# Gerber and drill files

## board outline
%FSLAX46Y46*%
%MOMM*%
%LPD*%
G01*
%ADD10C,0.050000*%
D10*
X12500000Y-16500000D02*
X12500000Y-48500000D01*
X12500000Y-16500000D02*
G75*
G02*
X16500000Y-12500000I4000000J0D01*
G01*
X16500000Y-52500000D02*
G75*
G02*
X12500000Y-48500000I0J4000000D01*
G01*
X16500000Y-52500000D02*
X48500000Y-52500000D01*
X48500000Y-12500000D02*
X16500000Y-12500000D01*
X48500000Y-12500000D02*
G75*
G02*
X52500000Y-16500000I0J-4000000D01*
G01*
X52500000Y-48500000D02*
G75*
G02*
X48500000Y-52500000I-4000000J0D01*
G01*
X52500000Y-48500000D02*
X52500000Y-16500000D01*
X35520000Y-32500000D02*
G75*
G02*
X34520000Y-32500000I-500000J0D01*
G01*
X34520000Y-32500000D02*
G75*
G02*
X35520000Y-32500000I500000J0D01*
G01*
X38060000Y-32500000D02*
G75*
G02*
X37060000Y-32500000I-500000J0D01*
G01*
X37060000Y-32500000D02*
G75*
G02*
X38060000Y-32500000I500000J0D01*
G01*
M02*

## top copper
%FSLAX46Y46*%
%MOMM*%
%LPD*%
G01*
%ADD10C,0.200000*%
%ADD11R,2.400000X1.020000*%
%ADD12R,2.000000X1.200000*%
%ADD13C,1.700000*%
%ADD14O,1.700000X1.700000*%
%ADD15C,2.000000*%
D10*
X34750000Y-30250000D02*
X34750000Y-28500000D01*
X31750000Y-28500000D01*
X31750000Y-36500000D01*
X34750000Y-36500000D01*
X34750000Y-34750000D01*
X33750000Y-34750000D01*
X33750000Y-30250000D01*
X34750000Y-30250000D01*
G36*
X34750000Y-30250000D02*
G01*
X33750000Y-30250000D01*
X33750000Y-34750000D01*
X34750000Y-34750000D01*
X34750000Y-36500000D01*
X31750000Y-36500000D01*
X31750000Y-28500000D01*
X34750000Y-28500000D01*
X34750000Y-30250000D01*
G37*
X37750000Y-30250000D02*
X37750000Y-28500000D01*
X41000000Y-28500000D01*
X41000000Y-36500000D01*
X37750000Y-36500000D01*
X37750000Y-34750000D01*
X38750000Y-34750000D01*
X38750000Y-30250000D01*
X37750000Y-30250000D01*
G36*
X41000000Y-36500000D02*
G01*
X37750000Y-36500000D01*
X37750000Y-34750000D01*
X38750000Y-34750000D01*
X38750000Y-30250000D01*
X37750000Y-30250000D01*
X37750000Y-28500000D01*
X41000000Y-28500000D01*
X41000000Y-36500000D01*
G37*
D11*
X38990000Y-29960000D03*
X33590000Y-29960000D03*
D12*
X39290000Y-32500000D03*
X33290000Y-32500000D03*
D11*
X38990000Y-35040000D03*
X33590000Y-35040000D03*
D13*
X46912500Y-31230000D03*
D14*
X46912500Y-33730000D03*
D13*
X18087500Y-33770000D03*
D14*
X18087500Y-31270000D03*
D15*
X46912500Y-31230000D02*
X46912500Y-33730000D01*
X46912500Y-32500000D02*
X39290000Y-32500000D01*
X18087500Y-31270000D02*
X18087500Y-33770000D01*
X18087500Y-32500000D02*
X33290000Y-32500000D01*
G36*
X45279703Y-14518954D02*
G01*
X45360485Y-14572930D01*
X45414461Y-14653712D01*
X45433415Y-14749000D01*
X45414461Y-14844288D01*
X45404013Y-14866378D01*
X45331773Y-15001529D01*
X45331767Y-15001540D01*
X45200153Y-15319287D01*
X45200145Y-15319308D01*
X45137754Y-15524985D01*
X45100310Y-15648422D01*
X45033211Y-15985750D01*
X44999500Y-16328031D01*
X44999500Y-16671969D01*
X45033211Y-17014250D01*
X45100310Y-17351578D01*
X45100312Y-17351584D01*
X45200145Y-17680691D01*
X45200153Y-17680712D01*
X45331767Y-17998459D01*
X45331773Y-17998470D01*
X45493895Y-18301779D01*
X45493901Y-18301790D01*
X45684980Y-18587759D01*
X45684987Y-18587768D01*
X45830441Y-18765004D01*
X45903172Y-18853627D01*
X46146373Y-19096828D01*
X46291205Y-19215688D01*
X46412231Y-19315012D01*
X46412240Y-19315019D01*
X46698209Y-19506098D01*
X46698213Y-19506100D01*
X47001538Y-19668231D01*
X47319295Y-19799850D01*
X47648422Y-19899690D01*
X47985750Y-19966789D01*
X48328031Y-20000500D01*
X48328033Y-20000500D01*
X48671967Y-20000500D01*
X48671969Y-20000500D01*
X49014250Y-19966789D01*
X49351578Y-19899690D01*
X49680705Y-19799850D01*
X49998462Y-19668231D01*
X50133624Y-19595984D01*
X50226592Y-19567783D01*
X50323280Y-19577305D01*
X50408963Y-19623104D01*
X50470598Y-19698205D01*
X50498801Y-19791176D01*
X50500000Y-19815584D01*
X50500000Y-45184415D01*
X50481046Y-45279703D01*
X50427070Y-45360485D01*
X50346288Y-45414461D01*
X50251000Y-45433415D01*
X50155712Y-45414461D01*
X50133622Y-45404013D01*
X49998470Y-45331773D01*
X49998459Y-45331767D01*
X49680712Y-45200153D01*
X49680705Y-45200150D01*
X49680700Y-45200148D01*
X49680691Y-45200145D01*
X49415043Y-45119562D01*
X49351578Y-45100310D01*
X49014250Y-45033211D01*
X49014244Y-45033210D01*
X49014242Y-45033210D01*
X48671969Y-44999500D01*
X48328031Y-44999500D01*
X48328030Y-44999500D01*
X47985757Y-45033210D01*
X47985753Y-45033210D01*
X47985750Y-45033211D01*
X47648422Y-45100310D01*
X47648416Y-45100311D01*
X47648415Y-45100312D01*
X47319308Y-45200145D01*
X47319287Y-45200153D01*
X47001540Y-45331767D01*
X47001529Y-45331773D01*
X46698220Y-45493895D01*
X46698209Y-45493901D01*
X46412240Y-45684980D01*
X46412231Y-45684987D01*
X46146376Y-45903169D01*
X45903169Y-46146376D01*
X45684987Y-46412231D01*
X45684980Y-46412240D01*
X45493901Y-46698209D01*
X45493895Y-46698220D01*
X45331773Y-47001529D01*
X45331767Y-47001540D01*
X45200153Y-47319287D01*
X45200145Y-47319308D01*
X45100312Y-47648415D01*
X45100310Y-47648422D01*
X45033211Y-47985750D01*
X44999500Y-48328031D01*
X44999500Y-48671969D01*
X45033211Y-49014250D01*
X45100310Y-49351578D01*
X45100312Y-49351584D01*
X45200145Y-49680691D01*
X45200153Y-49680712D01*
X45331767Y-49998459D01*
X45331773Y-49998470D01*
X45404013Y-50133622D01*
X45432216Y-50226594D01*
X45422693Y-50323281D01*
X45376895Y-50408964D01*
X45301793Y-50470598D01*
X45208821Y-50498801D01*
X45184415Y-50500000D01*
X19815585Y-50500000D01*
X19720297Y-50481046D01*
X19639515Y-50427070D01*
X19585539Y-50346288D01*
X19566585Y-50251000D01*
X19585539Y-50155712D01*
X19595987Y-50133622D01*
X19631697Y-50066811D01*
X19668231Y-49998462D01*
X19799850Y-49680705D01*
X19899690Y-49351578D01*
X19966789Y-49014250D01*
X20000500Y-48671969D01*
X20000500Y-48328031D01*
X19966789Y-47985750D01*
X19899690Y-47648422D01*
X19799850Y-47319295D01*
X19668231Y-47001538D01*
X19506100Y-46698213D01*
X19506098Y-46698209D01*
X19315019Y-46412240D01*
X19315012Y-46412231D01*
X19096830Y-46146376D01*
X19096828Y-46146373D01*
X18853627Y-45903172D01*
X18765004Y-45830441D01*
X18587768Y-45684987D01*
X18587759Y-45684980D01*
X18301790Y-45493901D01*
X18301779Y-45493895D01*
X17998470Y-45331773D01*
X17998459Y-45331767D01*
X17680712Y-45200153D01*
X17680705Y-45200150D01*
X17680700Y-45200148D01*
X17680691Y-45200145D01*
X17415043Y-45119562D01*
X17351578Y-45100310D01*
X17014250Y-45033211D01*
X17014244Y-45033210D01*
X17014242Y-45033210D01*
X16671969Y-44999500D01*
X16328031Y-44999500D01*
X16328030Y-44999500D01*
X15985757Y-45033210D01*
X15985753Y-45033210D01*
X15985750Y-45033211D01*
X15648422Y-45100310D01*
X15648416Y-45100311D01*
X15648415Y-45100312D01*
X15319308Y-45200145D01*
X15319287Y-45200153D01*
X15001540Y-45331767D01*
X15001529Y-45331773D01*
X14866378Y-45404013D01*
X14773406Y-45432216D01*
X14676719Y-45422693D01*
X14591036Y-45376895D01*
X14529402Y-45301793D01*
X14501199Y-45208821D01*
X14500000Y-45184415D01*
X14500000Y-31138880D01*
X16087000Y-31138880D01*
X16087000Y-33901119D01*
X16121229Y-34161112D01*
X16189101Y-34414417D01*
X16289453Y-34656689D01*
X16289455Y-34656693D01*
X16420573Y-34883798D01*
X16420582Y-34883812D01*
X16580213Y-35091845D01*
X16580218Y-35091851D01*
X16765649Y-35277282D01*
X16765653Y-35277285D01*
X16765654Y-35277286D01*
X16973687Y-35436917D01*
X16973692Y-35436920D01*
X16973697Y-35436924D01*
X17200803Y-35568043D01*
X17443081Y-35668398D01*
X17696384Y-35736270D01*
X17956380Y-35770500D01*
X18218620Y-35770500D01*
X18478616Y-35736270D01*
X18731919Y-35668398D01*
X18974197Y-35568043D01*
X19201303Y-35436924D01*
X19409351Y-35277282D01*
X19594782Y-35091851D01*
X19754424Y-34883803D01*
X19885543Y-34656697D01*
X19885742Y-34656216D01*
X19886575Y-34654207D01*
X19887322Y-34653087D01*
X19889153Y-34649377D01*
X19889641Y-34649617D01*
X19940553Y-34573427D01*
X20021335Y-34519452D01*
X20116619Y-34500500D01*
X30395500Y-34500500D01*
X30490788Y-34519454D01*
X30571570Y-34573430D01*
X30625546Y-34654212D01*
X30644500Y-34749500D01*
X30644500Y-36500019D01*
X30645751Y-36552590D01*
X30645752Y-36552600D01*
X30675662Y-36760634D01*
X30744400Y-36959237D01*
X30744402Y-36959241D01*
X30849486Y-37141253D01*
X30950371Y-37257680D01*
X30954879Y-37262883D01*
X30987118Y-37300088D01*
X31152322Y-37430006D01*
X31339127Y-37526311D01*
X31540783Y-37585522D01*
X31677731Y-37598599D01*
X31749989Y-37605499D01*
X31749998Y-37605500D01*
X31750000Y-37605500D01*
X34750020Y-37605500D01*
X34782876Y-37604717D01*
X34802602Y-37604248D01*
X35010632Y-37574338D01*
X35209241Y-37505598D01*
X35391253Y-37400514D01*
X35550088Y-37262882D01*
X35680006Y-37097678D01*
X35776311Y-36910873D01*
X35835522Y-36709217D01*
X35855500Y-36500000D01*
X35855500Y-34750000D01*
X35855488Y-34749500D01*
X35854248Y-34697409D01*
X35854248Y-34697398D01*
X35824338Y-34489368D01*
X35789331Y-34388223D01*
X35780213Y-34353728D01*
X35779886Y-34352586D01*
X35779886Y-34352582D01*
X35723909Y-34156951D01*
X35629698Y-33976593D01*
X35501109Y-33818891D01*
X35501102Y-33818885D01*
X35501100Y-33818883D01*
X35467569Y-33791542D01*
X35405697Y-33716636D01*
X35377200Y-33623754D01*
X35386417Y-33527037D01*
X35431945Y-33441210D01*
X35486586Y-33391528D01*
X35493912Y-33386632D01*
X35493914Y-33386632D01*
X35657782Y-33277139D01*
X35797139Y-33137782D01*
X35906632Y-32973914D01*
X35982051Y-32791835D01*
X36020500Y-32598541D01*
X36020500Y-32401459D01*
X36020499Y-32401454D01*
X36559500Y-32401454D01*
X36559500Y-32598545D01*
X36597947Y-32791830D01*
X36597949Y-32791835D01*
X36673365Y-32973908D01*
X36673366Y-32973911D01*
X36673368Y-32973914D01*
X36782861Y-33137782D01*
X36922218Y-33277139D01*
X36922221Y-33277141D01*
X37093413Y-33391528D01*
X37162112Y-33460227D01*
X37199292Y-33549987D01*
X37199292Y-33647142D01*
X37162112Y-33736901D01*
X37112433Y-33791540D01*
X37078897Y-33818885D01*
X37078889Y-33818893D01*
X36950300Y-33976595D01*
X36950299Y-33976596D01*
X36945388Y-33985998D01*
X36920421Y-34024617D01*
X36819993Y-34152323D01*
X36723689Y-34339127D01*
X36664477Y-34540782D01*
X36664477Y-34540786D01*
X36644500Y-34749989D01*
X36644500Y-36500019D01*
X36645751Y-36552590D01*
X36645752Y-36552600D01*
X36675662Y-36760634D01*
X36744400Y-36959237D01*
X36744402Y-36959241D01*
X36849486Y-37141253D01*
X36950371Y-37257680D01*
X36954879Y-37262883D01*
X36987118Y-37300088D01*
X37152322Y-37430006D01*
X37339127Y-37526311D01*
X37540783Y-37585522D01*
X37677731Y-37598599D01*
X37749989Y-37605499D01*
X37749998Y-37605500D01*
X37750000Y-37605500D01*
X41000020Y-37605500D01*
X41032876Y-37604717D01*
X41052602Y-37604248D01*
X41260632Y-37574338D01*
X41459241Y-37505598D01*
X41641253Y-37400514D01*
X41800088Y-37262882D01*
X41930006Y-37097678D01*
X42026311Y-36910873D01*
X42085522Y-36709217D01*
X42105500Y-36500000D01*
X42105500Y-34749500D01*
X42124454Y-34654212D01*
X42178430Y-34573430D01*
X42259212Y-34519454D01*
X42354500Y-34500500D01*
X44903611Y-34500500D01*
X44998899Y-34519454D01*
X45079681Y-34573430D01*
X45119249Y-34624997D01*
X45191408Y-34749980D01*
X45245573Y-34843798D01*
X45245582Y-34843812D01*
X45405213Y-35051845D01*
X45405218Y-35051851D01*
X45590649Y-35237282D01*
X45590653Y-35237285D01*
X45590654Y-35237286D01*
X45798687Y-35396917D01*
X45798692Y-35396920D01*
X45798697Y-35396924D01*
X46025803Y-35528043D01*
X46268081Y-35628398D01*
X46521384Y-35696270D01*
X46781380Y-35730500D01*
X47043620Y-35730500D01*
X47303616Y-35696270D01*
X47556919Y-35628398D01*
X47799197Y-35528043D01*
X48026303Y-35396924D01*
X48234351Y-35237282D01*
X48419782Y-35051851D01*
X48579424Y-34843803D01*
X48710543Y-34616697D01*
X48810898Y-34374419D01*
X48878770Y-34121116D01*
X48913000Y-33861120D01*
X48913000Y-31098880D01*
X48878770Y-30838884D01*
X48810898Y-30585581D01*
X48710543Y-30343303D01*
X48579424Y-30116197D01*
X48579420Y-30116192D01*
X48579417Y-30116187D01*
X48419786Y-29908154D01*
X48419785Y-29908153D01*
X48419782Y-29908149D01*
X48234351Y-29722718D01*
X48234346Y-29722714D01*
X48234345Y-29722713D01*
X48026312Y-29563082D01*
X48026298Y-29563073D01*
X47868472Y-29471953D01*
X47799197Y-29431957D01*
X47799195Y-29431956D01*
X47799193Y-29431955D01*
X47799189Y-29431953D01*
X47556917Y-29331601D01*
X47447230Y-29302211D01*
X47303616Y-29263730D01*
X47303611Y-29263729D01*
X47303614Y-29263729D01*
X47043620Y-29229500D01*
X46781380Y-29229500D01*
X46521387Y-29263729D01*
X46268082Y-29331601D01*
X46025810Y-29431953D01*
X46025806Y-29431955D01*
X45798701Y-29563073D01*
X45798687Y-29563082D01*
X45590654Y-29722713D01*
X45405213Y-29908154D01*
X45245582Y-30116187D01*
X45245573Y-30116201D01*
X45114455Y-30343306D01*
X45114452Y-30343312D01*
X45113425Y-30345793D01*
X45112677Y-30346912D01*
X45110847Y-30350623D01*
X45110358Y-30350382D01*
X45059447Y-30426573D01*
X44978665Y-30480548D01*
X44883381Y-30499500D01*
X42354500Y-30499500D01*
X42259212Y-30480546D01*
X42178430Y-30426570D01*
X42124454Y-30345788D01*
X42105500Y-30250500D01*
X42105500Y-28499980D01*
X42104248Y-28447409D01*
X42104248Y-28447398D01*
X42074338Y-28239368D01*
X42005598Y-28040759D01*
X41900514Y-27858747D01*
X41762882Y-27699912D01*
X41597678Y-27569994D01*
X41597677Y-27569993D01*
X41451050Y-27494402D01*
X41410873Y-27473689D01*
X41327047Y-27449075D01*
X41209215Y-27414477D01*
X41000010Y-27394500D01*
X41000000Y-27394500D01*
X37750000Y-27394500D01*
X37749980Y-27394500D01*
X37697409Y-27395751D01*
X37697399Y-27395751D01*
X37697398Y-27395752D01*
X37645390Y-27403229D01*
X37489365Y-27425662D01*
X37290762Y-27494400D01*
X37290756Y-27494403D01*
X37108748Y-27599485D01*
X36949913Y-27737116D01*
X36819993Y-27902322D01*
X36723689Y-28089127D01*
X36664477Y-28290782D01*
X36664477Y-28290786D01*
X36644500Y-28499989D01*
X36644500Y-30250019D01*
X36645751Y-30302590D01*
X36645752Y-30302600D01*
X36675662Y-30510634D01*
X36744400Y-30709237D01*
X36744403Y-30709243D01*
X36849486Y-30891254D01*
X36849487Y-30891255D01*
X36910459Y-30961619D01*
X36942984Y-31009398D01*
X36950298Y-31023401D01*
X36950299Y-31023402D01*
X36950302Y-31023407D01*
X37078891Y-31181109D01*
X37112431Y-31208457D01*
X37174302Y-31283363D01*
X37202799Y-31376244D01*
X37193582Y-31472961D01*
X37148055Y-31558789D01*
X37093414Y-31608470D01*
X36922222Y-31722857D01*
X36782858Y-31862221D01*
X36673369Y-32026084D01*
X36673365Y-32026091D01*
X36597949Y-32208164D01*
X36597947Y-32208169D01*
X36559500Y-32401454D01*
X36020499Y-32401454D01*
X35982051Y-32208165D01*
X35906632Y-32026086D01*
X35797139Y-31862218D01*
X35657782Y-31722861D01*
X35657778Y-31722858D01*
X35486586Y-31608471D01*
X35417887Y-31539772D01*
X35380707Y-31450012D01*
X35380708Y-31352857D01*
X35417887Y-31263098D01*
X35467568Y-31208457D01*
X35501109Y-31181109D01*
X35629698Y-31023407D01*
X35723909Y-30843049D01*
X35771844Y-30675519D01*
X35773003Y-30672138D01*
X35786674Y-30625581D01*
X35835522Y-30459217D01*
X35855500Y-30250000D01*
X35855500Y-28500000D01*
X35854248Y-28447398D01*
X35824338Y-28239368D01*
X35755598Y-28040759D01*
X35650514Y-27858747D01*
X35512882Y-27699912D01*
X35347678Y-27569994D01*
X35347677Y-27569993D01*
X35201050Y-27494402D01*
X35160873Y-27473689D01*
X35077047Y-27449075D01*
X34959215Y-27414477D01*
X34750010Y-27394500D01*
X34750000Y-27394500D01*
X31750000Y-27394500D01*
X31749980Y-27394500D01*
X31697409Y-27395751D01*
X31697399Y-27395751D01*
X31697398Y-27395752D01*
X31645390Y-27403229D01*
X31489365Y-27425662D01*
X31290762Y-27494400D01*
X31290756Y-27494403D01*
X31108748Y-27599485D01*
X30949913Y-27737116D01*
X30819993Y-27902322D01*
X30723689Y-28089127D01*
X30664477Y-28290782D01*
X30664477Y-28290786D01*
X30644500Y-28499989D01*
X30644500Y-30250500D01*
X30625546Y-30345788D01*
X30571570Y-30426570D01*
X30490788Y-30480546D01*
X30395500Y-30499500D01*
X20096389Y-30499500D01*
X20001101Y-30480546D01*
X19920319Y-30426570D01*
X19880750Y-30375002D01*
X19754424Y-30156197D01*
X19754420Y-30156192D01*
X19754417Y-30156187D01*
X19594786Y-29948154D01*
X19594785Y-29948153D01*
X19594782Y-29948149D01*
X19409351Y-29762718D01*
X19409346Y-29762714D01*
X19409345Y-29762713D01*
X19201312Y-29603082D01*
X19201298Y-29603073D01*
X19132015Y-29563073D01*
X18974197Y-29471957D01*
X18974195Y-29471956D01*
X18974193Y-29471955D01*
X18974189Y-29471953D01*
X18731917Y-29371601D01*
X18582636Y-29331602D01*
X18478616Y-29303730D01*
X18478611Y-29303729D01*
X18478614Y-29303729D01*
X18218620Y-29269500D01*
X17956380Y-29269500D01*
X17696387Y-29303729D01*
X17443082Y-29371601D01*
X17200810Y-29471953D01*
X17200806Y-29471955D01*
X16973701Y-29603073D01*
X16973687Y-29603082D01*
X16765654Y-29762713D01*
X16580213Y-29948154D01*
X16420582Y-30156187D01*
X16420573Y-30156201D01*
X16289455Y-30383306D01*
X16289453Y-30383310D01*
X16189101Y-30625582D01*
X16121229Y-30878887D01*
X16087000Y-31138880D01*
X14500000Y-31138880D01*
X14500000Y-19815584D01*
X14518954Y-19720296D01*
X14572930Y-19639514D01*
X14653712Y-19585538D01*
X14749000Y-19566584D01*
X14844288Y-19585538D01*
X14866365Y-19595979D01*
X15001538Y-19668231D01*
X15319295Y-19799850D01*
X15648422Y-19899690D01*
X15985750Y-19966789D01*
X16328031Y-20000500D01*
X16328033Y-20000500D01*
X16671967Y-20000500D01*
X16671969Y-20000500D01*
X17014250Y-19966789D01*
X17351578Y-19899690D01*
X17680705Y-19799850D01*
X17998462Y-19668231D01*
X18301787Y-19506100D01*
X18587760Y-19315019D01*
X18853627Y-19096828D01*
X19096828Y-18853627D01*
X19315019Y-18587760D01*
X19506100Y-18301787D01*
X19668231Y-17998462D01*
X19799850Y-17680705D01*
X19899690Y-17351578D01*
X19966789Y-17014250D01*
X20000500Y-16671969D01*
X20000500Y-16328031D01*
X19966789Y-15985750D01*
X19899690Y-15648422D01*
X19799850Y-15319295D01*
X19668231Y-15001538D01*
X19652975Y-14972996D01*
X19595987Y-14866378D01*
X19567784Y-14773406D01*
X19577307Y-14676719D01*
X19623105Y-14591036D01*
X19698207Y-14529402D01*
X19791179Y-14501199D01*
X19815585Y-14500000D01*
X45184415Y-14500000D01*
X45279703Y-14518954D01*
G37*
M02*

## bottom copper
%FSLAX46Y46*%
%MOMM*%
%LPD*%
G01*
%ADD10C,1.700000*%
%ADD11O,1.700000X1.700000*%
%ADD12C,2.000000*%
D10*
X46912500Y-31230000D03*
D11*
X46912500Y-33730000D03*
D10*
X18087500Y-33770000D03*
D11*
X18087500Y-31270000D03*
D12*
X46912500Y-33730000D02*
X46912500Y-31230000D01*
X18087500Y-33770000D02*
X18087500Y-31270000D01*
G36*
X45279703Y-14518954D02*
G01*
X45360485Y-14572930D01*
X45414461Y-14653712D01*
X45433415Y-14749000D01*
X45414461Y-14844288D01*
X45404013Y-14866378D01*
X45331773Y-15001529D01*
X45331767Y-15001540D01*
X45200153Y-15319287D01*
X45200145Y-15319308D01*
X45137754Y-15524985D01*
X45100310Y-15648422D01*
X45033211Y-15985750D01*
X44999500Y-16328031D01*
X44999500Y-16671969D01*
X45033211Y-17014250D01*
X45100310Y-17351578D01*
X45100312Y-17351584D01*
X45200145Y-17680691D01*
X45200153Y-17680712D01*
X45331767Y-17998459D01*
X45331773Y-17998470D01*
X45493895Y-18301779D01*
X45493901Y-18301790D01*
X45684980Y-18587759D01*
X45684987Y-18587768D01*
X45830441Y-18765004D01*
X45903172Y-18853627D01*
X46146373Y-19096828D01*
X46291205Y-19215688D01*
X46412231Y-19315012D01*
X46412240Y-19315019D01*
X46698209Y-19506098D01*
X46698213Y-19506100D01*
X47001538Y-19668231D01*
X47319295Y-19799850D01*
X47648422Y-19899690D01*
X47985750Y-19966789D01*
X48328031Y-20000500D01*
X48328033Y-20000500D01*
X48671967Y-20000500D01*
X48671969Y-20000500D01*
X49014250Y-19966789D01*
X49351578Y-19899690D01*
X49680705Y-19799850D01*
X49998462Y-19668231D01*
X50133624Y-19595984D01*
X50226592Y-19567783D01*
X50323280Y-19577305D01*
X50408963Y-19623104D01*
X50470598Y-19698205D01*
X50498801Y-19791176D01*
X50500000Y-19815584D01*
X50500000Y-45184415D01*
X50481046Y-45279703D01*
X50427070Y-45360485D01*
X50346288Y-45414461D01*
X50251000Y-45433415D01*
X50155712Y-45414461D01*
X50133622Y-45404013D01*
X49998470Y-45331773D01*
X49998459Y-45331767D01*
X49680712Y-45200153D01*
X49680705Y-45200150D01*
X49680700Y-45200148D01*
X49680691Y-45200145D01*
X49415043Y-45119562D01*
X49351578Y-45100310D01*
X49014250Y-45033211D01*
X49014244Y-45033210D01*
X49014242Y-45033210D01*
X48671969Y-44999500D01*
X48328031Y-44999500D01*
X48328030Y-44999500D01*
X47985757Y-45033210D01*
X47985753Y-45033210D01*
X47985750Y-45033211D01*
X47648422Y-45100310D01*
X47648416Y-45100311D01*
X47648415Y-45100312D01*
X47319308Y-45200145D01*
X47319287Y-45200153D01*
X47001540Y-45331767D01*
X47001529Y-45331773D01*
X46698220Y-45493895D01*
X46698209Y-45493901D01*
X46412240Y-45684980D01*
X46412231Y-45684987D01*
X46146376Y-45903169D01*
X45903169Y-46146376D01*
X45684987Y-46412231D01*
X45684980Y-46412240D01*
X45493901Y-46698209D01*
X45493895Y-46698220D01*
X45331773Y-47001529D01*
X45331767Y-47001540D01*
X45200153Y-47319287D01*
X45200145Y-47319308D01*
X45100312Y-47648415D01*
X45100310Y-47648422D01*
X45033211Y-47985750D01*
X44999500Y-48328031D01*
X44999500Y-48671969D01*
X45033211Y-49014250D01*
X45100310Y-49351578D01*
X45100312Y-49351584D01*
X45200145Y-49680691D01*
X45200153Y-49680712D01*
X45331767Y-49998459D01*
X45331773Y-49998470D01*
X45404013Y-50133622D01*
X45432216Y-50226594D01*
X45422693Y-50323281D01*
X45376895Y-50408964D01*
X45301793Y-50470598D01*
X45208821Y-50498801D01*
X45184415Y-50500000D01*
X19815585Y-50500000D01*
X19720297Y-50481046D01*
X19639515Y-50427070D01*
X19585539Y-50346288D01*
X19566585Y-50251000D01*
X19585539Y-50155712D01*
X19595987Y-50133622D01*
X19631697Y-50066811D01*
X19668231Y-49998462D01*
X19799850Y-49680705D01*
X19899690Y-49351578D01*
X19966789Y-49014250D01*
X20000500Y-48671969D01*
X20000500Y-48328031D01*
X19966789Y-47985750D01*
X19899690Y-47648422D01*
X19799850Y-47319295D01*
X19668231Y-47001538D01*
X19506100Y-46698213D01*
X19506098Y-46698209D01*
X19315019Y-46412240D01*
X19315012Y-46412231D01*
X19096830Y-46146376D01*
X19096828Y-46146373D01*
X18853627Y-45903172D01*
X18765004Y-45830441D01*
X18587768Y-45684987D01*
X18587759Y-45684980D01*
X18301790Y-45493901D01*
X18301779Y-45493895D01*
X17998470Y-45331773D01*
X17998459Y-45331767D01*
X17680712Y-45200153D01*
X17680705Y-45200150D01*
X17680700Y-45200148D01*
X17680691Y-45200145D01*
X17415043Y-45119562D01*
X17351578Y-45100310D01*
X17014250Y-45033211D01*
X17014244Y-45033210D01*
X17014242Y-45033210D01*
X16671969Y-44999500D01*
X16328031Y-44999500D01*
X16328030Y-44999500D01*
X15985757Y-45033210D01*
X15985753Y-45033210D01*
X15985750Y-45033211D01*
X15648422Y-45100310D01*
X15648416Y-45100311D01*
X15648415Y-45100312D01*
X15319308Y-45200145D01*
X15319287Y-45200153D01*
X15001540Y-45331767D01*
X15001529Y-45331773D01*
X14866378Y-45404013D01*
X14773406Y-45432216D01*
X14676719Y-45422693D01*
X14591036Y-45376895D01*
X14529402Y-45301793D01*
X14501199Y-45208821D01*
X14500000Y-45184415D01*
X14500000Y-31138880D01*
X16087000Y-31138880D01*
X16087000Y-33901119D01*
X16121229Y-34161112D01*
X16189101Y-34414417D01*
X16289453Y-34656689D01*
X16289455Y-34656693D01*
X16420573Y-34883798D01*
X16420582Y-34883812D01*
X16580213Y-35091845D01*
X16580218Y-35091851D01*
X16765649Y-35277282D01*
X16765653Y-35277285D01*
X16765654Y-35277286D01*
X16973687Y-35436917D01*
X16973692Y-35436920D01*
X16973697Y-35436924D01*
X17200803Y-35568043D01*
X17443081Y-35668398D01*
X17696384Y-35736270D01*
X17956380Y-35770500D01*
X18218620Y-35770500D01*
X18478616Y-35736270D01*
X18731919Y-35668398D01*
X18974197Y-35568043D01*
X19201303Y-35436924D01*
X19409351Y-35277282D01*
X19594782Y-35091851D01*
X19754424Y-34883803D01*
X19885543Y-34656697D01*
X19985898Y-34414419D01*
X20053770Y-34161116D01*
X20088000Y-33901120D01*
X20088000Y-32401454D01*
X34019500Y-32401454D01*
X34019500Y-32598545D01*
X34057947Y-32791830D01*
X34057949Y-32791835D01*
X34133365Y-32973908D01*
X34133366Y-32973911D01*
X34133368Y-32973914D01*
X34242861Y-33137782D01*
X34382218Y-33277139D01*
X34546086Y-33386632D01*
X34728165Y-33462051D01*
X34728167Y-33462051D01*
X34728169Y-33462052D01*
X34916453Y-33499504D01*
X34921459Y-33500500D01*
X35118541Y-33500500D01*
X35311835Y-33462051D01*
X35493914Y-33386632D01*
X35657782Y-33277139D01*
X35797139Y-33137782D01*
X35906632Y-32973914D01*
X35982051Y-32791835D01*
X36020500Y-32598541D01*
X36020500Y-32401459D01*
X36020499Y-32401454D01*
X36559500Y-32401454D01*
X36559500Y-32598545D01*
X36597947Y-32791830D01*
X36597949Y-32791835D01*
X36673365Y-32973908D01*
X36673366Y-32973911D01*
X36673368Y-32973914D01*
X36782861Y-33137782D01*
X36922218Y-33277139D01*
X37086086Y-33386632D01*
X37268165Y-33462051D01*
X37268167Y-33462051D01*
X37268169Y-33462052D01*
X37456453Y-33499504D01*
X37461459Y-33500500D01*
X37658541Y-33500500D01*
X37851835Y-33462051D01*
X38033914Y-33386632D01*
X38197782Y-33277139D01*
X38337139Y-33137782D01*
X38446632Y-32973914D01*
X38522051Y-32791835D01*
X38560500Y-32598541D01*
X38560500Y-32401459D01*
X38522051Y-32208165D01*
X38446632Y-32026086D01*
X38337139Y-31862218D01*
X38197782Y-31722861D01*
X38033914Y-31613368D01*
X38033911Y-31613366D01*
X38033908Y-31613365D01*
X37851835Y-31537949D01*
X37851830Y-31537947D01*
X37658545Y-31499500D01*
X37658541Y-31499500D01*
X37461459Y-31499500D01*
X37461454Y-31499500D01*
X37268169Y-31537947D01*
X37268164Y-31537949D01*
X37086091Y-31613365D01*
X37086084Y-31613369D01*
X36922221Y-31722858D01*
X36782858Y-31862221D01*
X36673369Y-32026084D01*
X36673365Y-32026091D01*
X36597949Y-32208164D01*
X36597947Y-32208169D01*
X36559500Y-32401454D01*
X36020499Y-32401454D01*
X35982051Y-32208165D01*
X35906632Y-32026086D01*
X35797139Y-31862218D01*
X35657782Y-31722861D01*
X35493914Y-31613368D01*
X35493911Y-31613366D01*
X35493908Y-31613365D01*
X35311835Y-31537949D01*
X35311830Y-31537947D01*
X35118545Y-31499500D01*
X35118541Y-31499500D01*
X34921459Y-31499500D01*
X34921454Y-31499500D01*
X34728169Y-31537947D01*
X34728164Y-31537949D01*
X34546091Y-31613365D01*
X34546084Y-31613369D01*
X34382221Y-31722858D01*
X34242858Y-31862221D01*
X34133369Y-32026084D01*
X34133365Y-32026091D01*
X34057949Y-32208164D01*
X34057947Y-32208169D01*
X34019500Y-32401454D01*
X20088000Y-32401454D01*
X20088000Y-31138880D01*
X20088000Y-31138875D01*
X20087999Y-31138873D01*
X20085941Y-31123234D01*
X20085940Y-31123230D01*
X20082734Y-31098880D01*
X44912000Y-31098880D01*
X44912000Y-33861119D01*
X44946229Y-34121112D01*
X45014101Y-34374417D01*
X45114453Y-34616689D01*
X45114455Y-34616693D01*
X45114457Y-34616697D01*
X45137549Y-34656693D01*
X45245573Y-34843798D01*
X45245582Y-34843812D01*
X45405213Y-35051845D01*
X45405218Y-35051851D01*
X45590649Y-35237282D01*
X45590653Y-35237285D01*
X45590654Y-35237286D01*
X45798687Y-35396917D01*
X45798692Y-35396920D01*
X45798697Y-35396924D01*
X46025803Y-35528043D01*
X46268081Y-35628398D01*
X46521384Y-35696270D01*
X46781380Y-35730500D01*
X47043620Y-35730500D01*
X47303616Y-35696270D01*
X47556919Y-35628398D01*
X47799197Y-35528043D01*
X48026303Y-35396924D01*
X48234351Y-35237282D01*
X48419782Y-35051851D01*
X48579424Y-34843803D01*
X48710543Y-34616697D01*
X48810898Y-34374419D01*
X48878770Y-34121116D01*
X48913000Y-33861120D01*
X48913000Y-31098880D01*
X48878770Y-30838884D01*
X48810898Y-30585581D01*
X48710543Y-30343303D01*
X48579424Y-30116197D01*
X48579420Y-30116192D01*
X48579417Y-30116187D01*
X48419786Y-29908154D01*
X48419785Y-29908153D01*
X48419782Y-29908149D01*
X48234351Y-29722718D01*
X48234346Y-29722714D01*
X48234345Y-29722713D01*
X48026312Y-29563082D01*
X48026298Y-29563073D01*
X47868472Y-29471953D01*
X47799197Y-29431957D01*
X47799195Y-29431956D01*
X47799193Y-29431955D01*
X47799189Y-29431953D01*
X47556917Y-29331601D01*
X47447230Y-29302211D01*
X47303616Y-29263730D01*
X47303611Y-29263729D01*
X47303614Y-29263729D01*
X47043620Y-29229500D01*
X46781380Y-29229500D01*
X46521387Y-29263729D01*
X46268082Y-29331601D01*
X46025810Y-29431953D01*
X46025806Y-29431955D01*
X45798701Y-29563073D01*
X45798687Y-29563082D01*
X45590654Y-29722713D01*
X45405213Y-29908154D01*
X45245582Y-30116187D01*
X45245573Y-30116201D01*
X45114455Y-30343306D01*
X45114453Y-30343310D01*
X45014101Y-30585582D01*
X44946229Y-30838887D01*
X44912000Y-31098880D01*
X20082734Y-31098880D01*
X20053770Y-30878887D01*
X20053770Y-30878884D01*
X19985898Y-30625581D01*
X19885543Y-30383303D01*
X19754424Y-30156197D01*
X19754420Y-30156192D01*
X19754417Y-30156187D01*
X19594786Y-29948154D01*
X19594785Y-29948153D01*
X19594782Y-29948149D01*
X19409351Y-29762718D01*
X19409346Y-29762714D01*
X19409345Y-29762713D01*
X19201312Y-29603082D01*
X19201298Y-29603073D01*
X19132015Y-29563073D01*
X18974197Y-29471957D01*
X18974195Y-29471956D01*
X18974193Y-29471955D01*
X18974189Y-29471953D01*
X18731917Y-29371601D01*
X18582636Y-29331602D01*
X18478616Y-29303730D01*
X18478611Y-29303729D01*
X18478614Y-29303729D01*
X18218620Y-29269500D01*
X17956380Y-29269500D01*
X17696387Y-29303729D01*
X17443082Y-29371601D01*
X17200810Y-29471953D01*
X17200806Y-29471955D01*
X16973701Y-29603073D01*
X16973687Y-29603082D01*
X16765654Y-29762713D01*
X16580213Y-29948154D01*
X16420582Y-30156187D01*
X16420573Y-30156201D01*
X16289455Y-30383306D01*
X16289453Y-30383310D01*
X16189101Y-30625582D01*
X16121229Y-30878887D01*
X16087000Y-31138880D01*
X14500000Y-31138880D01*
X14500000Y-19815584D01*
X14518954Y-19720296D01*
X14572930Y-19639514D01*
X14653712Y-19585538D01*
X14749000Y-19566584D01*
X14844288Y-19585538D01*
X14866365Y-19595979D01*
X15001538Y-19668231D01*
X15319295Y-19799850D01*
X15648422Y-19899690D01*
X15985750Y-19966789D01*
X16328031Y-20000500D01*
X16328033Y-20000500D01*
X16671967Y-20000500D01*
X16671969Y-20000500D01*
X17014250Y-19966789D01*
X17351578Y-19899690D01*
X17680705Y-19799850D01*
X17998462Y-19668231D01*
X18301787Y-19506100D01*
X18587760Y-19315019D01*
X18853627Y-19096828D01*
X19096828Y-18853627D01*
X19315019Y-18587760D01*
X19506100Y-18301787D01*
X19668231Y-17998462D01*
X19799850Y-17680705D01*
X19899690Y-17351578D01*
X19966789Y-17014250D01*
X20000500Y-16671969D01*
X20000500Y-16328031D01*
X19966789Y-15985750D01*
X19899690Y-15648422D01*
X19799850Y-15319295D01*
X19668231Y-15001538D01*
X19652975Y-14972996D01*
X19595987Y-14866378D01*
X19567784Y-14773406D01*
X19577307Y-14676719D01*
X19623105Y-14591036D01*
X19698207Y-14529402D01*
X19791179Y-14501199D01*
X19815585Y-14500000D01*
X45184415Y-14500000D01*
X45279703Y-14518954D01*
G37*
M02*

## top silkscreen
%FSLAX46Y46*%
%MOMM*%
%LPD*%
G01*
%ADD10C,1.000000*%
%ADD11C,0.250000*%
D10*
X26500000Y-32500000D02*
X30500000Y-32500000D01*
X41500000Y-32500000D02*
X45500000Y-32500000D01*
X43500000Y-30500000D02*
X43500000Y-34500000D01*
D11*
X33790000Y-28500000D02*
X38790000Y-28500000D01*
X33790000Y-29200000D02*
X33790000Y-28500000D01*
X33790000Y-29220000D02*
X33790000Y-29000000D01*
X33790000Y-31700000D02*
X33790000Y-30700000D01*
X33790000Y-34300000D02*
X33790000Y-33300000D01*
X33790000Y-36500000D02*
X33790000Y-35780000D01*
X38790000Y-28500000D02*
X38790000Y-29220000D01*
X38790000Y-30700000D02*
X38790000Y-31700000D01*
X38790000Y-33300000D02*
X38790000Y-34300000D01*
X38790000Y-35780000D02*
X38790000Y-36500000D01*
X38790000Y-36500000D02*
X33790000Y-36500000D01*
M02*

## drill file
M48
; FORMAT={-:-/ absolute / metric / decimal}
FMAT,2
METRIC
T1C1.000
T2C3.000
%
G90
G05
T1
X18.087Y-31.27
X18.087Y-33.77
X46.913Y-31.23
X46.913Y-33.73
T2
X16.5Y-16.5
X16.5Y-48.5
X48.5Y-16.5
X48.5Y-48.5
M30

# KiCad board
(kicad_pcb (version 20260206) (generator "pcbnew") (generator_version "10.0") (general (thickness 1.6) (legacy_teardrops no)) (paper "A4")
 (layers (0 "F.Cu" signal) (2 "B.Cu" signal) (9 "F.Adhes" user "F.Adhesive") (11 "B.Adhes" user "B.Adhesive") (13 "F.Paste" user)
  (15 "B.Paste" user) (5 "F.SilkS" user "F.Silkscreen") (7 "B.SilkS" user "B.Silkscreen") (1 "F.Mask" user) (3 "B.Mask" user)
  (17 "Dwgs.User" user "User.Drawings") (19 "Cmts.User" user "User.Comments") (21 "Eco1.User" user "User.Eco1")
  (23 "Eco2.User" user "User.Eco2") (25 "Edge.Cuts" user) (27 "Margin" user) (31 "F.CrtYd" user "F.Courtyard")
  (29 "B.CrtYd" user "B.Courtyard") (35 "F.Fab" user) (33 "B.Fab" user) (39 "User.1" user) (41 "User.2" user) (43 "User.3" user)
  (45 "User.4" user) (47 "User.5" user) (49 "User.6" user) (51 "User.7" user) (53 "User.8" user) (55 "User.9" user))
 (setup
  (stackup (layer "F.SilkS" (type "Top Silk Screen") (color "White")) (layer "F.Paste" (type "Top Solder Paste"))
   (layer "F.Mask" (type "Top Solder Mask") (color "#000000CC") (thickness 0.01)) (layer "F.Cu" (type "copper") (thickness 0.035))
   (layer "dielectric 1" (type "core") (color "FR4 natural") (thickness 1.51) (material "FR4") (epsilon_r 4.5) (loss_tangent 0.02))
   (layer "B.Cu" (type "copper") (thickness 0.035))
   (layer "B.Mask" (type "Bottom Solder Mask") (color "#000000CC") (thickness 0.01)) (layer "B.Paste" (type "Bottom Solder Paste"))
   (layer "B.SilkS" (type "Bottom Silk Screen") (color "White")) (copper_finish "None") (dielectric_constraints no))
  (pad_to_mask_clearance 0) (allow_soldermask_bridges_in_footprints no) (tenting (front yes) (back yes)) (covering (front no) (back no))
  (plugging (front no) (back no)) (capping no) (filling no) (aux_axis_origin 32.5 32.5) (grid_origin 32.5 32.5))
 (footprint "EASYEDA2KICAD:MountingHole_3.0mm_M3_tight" (layer "F.Cu") (at 16.5 16.5 90)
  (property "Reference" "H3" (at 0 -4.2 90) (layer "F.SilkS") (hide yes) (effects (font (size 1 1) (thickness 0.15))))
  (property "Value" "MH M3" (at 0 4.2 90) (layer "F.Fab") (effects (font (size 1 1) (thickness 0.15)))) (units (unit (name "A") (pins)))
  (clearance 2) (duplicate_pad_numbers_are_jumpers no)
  (pad "" np_thru_hole circle (at 0 0 90) (size 3 3) (drill 3) (layers "*.Cu" "*.Mask")))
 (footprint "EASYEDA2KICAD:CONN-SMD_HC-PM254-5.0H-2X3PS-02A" (layer "F.Cu") (at 36.29 32.5 -90)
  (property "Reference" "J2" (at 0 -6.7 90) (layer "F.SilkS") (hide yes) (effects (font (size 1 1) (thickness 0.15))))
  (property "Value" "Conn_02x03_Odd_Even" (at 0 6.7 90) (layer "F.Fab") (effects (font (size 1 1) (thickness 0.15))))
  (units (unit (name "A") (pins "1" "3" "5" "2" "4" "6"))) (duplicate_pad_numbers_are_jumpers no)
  (fp_line (start -4 2.5) (end -4 -2.5) (stroke (width 0.25) (type solid)) (layer "F.SilkS"))
  (fp_line (start -3.3 2.5) (end -4 2.5) (stroke (width 0.25) (type solid)) (layer "F.SilkS"))
  (fp_line (start -3.28 2.5) (end -3.5 2.5) (stroke (width 0.25) (type solid)) (layer "F.SilkS"))
  (fp_line (start -0.8 2.5) (end -1.8 2.5) (stroke (width 0.25) (type solid)) (layer "F.SilkS"))
  (fp_line (start 1.8 2.5) (end 0.8 2.5) (stroke (width 0.25) (type solid)) (layer "F.SilkS"))
  (fp_line (start 4 2.5) (end 3.28 2.5) (stroke (width 0.25) (type solid)) (layer "F.SilkS"))
  (fp_line (start -4 -2.5) (end -3.28 -2.5) (stroke (width 0.25) (type solid)) (layer "F.SilkS"))
  (fp_line (start -1.8 -2.5) (end -0.8 -2.5) (stroke (width 0.25) (type solid)) (layer "F.SilkS"))
  (fp_line (start 0.8 -2.5) (end 1.8 -2.5) (stroke (width 0.25) (type solid)) (layer "F.SilkS"))
  (fp_line (start 3.28 -2.5) (end 4 -2.5) (stroke (width 0.25) (type solid)) (layer "F.SilkS"))
  (fp_line (start 4 -2.5) (end 4 2.5) (stroke (width 0.25) (type solid)) (layer "F.SilkS"))
  (fp_circle (center 0 1.27) (end 0.5 1.27) (stroke (width 0.05) (type default)) (fill no) (layer "Edge.Cuts"))
  (fp_circle (center 0 -1.27) (end 0.5 -1.27) (stroke (width 0.05) (type default)) (fill no) (layer "Edge.Cuts"))
  (pad "1" smd rect (at -2.54 -2.7 270) (size 1.02 2.4) (layers "F.Cu" "F.Mask" "F.Paste") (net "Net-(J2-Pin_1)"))
  (pad "2" smd rect (at -2.54 2.7 270) (size 1.02 2.4) (layers "F.Cu" "F.Mask" "F.Paste") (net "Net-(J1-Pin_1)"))
  (pad "3" smd rect (at 0 -3 90) (size 1.2 2) (layers "F.Cu" "F.Mask" "F.Paste") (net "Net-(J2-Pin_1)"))
  (pad "4" smd rect (at 0 3 90) (size 1.2 2) (layers "F.Cu" "F.Mask" "F.Paste") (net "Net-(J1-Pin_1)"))
  (pad "5" smd rect (at 2.54 -2.7 270) (size 1.02 2.4) (layers "F.Cu" "F.Mask" "F.Paste") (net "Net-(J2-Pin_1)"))
  (pad "6" smd rect (at 2.54 2.7 270) (size 1.02 2.4) (layers "F.Cu" "F.Mask" "F.Paste") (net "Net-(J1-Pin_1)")))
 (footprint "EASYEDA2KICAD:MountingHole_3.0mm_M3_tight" (layer "F.Cu") (at 16.5 48.5 90)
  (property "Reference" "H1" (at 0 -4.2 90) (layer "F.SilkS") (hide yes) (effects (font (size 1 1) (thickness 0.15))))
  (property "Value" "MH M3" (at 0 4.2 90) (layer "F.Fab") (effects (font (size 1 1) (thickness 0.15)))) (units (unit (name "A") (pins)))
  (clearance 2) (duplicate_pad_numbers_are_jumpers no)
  (pad "" np_thru_hole circle (at 0 0 90) (size 3 3) (drill 3) (layers "*.Cu" "*.Mask")))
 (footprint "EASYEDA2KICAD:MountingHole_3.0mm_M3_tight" (layer "F.Cu") (at 48.5 16.5 90)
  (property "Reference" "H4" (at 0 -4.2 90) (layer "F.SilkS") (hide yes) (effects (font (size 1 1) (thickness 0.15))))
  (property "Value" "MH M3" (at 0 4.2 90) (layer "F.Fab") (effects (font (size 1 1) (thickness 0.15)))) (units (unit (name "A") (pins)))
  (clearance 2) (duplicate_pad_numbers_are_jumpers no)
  (pad "" np_thru_hole circle (at 0 0 90) (size 3 3) (drill 3) (layers "*.Cu" "*.Mask")))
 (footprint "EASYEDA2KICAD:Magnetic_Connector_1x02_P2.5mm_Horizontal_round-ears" (layer "F.Cu") (at 47.0125 32.5)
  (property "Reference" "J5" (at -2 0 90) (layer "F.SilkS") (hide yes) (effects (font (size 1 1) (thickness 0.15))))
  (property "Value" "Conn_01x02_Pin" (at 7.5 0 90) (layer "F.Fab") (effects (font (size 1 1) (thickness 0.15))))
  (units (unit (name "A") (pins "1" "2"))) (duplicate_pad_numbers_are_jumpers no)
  (pad "1" thru_hole circle (at -0.1 -1.27) (size 1.7 1.7) (drill 1) (layers "*.Cu" "*.Mask") (remove_unused_layers no)
   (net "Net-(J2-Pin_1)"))
  (pad "2" thru_hole oval (at -0.1 1.23) (size 1.7 1.7) (drill 1) (layers "*.Cu" "*.Mask") (remove_unused_layers no) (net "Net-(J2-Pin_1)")))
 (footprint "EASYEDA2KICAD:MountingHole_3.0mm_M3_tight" (layer "F.Cu") (at 48.5 48.5 90)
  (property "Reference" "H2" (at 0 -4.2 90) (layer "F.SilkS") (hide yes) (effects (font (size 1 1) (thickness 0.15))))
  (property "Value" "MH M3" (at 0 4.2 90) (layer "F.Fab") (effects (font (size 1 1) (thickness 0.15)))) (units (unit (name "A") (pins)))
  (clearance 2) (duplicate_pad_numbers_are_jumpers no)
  (pad "" np_thru_hole circle (at 0 0 90) (size 3 3) (drill 3) (layers "*.Cu" "*.Mask")))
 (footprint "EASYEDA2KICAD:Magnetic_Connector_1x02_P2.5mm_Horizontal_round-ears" (layer "F.Cu") (at 17.9875 32.5 180)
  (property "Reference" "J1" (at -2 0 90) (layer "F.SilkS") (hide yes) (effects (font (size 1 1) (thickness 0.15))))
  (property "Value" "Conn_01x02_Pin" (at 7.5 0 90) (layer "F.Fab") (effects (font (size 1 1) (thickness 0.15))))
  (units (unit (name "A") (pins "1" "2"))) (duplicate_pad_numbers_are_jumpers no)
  (pad "1" thru_hole circle (at -0.1 -1.27 180) (size 1.7 1.7) (drill 1) (layers "*.Cu" "*.Mask") (remove_unused_layers no)
   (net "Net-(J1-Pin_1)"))
  (pad "2" thru_hole oval (at -0.1 1.23 180) (size 1.7 1.7) (drill 1) (layers "*.Cu" "*.Mask") (remove_unused_layers no)
   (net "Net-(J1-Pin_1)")))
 (gr_poly
  (pts (xy 34.75 30.25) (xy 34.75 28.5) (xy 31.75 28.5) (xy 31.75 36.5) (xy 34.75 36.5) (xy 34.75 34.75) (xy 33.75 34.75) (xy 33.75 30.25))
  (stroke (width 0.2) (type solid)) (fill yes) (layer "F.Cu") (net "Net-(J1-Pin_1)"))
 (gr_poly
  (pts (xy 37.75 30.25) (xy 37.75 28.5) (xy 41 28.5) (xy 41 36.5) (xy 37.75 36.5) (xy 37.75 34.75) (xy 38.75 34.75) (xy 38.75 30.25))
  (stroke (width 0.2) (type solid)) (fill yes) (layer "F.Cu") (net "Net-(J2-Pin_1)"))
 (gr_line (start 26.5 32.5) (end 30.5 32.5) (stroke (width 1) (type default)) (layer "F.SilkS"))
 (gr_line (start 41.5 32.5) (end 45.5 32.5) (stroke (width 1) (type default)) (layer "F.SilkS"))
 (gr_line (start 43.5 30.5) (end 43.5 34.5) (stroke (width 1) (type default)) (layer "F.SilkS"))
 (gr_line (start 12.5 16.5) (end 12.5 48.5) (stroke (width 0.05) (type default)) (layer "Edge.Cuts"))
 (gr_arc (start 12.5 16.5) (mid 13.671573 13.671573) (end 16.5 12.5) (stroke (width 0.05) (type default)) (layer "Edge.Cuts"))
 (gr_arc (start 16.5 52.5) (mid 13.671573 51.328427) (end 12.5 48.5) (stroke (width 0.05) (type default)) (layer "Edge.Cuts"))
 (gr_line (start 16.5 52.5) (end 48.5 52.5) (stroke (width 0.05) (type default)) (layer "Edge.Cuts"))
 (gr_line (start 48.5 12.5) (end 16.5 12.5) (stroke (width 0.05) (type default)) (layer "Edge.Cuts"))
 (gr_arc (start 48.5 12.5) (mid 51.328427 13.671573) (end 52.5 16.5) (stroke (width 0.05) (type default)) (layer "Edge.Cuts"))
 (gr_arc (start 52.5 48.5) (mid 51.328427 51.328427) (end 48.5 52.5) (stroke (width 0.05) (type default)) (layer "Edge.Cuts"))
 (gr_line (start 52.5 48.5) (end 52.5 16.5) (stroke (width 0.05) (type default)) (layer "Edge.Cuts"))
 (segment (start 46.9125 31.23) (end 46.9125 33.73) (width 2) (layer "F.Cu") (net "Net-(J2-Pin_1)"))
 (segment (start 46.9125 32.5) (end 39.29 32.5) (width 2) (layer "F.Cu") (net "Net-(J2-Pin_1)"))
 (segment (start 46.9125 33.73) (end 46.9125 31.23) (width 2) (layer "B.Cu") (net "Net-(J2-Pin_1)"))
 (segment (start 18.0875 31.27) (end 18.0875 33.77) (width 2) (layer "F.Cu") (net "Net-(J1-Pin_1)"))
 (segment (start 18.0875 32.5) (end 33.29 32.5) (width 2) (layer "F.Cu") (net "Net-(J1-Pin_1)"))
 (segment (start 18.0875 33.77) (end 18.0875 31.27) (width 2) (layer "B.Cu") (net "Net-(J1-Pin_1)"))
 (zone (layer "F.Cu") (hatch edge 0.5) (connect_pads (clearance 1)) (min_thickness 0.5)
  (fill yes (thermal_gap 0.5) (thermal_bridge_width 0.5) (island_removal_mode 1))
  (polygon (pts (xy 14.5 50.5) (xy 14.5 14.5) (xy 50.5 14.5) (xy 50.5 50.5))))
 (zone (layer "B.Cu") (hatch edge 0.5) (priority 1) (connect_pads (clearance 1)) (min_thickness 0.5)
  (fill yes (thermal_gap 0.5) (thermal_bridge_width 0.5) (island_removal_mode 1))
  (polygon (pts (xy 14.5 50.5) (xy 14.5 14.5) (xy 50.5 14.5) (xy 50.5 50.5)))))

